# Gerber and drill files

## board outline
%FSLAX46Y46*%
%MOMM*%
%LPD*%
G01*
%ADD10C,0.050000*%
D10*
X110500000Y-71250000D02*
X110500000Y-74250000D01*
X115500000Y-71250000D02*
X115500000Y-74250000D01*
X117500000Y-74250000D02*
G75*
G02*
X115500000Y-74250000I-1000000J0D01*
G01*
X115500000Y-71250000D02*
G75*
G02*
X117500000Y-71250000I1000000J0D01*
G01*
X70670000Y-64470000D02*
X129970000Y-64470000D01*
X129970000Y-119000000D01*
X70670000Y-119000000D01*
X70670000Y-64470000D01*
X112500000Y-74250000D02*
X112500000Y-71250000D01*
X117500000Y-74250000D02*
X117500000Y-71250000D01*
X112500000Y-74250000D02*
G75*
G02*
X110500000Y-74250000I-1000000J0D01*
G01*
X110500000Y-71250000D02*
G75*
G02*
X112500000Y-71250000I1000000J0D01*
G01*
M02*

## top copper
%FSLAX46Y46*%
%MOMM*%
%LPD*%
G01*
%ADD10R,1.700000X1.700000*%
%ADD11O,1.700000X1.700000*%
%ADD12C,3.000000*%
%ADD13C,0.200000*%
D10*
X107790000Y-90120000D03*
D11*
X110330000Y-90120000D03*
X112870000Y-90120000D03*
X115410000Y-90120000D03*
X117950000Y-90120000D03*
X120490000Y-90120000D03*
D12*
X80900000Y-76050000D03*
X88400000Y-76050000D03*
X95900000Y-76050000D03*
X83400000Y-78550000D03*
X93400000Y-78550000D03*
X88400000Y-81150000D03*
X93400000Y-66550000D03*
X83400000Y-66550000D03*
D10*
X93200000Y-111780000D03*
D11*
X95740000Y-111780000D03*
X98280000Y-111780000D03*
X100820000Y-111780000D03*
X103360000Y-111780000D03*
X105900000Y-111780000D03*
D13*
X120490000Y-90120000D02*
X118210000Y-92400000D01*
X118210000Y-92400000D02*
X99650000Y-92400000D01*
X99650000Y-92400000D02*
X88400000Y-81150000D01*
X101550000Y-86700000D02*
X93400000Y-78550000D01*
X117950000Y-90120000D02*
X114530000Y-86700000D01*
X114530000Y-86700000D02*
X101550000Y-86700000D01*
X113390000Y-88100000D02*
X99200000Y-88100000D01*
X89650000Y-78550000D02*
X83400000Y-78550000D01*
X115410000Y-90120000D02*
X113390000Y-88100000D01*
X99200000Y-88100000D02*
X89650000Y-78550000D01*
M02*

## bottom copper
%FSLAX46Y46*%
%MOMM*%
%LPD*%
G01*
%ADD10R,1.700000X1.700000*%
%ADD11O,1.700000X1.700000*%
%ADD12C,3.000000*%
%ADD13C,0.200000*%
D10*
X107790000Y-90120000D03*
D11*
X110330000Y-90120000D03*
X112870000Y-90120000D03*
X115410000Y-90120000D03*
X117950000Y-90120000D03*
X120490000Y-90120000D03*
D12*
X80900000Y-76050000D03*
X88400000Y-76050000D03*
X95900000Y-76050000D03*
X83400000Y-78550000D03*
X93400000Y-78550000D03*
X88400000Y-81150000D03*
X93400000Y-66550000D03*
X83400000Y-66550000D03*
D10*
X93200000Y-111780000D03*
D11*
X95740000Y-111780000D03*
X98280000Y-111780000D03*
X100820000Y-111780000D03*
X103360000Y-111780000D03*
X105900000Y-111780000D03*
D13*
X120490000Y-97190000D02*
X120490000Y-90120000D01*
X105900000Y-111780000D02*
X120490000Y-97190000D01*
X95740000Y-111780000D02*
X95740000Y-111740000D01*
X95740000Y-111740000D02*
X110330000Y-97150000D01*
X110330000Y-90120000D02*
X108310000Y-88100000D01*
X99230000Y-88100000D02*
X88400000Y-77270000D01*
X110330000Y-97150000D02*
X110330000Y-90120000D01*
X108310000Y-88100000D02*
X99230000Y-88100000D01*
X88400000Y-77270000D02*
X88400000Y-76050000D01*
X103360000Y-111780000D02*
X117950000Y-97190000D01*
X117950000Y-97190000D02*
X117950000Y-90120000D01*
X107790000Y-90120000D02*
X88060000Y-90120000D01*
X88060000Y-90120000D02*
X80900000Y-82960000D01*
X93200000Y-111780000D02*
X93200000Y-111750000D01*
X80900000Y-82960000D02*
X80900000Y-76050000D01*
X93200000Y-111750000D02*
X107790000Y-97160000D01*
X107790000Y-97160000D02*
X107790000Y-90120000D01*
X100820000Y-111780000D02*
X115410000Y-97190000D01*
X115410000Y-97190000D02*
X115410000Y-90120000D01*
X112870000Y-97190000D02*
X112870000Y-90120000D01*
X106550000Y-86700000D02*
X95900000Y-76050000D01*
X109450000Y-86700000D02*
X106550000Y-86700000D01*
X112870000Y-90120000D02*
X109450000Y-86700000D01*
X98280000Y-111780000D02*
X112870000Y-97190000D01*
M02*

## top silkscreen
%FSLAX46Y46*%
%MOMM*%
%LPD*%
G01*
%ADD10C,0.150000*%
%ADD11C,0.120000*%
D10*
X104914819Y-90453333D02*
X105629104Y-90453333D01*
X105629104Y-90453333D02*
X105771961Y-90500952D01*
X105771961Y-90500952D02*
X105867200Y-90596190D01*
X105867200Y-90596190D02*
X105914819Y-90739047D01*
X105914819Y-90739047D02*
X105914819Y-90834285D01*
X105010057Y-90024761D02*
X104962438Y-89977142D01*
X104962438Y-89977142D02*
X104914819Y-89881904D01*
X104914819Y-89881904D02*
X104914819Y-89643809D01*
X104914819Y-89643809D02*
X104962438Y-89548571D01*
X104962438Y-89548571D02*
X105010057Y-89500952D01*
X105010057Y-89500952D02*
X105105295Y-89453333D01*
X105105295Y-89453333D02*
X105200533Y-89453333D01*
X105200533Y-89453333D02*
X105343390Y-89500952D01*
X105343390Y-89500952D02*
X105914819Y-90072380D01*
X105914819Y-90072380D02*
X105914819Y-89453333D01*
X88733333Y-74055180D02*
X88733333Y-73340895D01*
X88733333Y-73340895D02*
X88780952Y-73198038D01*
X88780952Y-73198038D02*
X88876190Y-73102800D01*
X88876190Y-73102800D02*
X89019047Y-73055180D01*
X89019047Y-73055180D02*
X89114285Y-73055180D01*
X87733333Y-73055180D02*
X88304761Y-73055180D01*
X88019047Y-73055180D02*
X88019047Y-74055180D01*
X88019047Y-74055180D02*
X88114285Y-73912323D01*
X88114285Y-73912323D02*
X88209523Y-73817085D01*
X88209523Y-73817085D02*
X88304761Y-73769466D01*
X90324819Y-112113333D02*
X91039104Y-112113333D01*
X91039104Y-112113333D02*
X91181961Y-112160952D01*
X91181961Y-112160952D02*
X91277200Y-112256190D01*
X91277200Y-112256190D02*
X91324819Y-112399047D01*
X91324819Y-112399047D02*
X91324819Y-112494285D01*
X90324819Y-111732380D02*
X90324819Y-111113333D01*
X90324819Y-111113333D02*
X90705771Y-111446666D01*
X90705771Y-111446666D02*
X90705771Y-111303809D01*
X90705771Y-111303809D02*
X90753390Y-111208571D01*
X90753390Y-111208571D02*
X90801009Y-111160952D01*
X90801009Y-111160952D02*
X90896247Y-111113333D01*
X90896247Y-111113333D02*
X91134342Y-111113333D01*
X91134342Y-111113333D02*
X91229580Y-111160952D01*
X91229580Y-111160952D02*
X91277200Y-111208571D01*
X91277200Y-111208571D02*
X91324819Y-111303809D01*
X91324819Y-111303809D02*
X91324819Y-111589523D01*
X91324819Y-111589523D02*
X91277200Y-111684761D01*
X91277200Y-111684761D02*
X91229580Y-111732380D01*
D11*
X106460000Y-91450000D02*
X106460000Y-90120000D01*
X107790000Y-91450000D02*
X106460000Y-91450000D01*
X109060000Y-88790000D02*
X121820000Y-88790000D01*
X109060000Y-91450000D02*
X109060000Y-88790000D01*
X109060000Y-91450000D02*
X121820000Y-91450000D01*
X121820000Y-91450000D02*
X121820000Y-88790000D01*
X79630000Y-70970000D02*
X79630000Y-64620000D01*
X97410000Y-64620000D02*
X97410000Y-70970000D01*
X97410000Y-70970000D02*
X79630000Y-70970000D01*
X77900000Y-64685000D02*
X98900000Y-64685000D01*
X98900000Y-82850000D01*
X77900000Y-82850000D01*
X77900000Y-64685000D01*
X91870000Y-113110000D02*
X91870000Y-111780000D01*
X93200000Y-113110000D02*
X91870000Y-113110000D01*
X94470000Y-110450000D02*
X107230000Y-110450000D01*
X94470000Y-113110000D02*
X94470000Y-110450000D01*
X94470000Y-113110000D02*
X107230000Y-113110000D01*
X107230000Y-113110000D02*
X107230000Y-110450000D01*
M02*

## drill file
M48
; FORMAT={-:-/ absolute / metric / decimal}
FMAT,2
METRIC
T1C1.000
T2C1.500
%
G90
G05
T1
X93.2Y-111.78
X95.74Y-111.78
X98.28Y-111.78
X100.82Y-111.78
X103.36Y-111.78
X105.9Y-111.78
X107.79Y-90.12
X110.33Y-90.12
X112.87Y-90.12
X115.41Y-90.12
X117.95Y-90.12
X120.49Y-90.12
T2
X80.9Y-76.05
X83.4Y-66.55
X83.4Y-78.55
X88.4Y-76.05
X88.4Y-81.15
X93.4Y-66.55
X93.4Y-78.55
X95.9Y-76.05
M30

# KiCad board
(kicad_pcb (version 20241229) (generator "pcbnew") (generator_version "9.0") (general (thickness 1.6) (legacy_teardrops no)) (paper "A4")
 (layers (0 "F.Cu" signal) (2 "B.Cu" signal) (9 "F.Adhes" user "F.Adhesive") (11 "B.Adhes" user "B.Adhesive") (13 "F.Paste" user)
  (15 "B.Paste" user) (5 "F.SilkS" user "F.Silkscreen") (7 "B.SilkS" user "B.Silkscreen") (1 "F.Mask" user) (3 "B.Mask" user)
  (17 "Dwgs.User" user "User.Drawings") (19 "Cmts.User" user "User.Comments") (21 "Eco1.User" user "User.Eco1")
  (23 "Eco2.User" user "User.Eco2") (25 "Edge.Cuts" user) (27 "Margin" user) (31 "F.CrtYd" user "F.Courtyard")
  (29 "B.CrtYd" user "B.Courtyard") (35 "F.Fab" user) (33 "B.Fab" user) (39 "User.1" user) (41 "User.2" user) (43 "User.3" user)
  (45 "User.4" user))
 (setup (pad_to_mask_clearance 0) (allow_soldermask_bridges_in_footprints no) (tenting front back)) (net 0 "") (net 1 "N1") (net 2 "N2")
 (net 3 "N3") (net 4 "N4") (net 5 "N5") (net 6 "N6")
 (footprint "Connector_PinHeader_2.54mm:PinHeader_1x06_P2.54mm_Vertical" (layer "F.Cu") (at 107.79 90.12 90)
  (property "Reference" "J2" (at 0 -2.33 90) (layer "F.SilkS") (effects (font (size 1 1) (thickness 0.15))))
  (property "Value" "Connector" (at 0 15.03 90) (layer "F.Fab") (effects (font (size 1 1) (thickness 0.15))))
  (fp_line (start -1.33 -1.33) (end 0 -1.33) (stroke (width 0.12) (type solid)) (layer "F.SilkS"))
  (fp_line (start -1.33 0) (end -1.33 -1.33) (stroke (width 0.12) (type solid)) (layer "F.SilkS"))
  (fp_line (start 1.33 1.27) (end 1.33 14.03) (stroke (width 0.12) (type solid)) (layer "F.SilkS"))
  (fp_line (start -1.33 1.27) (end 1.33 1.27) (stroke (width 0.12) (type solid)) (layer "F.SilkS"))
  (fp_line (start -1.33 1.27) (end -1.33 14.03) (stroke (width 0.12) (type solid)) (layer "F.SilkS"))
  (fp_line (start -1.33 14.03) (end 1.33 14.03) (stroke (width 0.12) (type solid)) (layer "F.SilkS"))
  (pad "1" thru_hole rect (at 0 0 90) (size 1.7 1.7) (drill 1) (layers "*.Cu" "*.Mask") (remove_unused_layers no) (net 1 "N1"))
  (pad "2" thru_hole oval (at 0 2.54 90) (size 1.7 1.7) (drill 1) (layers "*.Cu" "*.Mask") (remove_unused_layers no) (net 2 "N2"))
  (pad "3" thru_hole oval (at 0 5.08 90) (size 1.7 1.7) (drill 1) (layers "*.Cu" "*.Mask") (remove_unused_layers no) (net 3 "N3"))
  (pad "4" thru_hole oval (at 0 7.62 90) (size 1.7 1.7) (drill 1) (layers "*.Cu" "*.Mask") (remove_unused_layers no) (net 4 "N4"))
  (pad "5" thru_hole oval (at 0 10.16 90) (size 1.7 1.7) (drill 1) (layers "*.Cu" "*.Mask") (remove_unused_layers no) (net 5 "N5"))
  (pad "6" thru_hole oval (at 0 12.7 90) (size 1.7 1.7) (drill 1) (layers "*.Cu" "*.Mask") (remove_unused_layers no) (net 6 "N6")))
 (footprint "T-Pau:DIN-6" (layer "F.Cu") (at 80.9 76.05 180)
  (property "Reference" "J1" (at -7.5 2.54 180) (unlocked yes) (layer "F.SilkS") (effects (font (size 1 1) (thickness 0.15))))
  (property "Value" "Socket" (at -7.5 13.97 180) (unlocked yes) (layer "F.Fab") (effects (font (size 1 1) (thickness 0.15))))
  (fp_line (start 1.27 5.08) (end 1.27 11.43) (stroke (width 0.12) (type default)) (layer "F.SilkS"))
  (fp_line (start -16.51 11.43) (end -16.51 5.08) (stroke (width 0.12) (type default)) (layer "F.SilkS"))
  (fp_line (start -16.51 5.08) (end 1.27 5.08) (stroke (width 0.12) (type default)) (layer "F.SilkS"))
  (fp_rect (start -18 -6.8) (end 3 11.365) (stroke (width 0.12) (type default)) (fill no) (layer "F.SilkS"))
  (pad "1" thru_hole circle (at 0 0 180) (size 3 3) (drill 1.5) (layers "*.Cu" "*.Mask") (remove_unused_layers no) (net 1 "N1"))
  (pad "2" thru_hole circle (at -7.5 0 180) (size 3 3) (drill 1.5) (layers "*.Cu" "*.Mask") (remove_unused_layers no) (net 2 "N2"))
  (pad "3" thru_hole circle (at -15 0 180) (size 3 3) (drill 1.5) (layers "*.Cu" "*.Mask") (remove_unused_layers no) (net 3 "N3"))
  (pad "4" thru_hole circle (at -2.5 -2.5 180) (size 3 3) (drill 1.5) (layers "*.Cu" "*.Mask") (remove_unused_layers no) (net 4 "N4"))
  (pad "5" thru_hole circle (at -12.5 -2.5 180) (size 3 3) (drill 1.5) (layers "*.Cu" "*.Mask") (remove_unused_layers no) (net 5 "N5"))
  (pad "6" thru_hole circle (at -7.5 -5.1 180) (size 3 3) (drill 1.5) (layers "*.Cu" "*.Mask") (remove_unused_layers no) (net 6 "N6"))
  (pad "7" thru_hole circle (at -12.5 9.5 180) (size 3 3) (drill 1.5) (layers "*.Cu" "*.Mask") (remove_unused_layers no))
  (pad "7" thru_hole circle (at -2.5 9.5 180) (size 3 3) (drill 1.5) (layers "*.Cu" "*.Mask") (remove_unused_layers no)))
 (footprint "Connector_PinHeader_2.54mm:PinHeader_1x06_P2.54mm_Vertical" (layer "F.Cu") (at 93.2 111.78 90)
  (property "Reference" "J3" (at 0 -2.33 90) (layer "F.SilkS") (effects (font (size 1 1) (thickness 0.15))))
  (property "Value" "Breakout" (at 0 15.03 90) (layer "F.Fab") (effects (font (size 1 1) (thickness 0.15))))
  (fp_line (start -1.33 -1.33) (end 0 -1.33) (stroke (width 0.12) (type solid)) (layer "F.SilkS"))
  (fp_line (start -1.33 0) (end -1.33 -1.33) (stroke (width 0.12) (type solid)) (layer "F.SilkS"))
  (fp_line (start 1.33 1.27) (end 1.33 14.03) (stroke (width 0.12) (type solid)) (layer "F.SilkS"))
  (fp_line (start -1.33 1.27) (end 1.33 1.27) (stroke (width 0.12) (type solid)) (layer "F.SilkS"))
  (fp_line (start -1.33 1.27) (end -1.33 14.03) (stroke (width 0.12) (type solid)) (layer "F.SilkS"))
  (fp_line (start -1.33 14.03) (end 1.33 14.03) (stroke (width 0.12) (type solid)) (layer "F.SilkS"))
  (pad "1" thru_hole rect (at 0 0 90) (size 1.7 1.7) (drill 1) (layers "*.Cu" "*.Mask") (remove_unused_layers no) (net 1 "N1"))
  (pad "2" thru_hole oval (at 0 2.54 90) (size 1.7 1.7) (drill 1) (layers "*.Cu" "*.Mask") (remove_unused_layers no) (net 2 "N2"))
  (pad "3" thru_hole oval (at 0 5.08 90) (size 1.7 1.7) (drill 1) (layers "*.Cu" "*.Mask") (remove_unused_layers no) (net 3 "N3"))
  (pad "4" thru_hole oval (at 0 7.62 90) (size 1.7 1.7) (drill 1) (layers "*.Cu" "*.Mask") (remove_unused_layers no) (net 4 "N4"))
  (pad "5" thru_hole oval (at 0 10.16 90) (size 1.7 1.7) (drill 1) (layers "*.Cu" "*.Mask") (remove_unused_layers no) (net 5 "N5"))
  (pad "6" thru_hole oval (at 0 12.7 90) (size 1.7 1.7) (drill 1) (layers "*.Cu" "*.Mask") (remove_unused_layers no) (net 6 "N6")))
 (gr_line (start 110.5 71.25) (end 110.5 74.25) (stroke (width 0.05) (type default)) (layer "Edge.Cuts"))
 (gr_line (start 115.5 71.25) (end 115.5 74.25) (stroke (width 0.05) (type default)) (layer "Edge.Cuts"))
 (gr_arc (start 117.5 74.25) (mid 116.5 75.25) (end 115.5 74.25) (stroke (width 0.05) (type default)) (layer "Edge.Cuts"))
 (gr_arc (start 115.5 71.25) (mid 116.5 70.25) (end 117.5 71.25) (stroke (width 0.05) (type default)) (layer "Edge.Cuts"))
 (gr_rect (start 70.67 64.47) (end 129.97 119) (stroke (width 0.05) (type default)) (fill no) (layer "Edge.Cuts"))
 (gr_line (start 112.5 74.25) (end 112.5 71.25) (stroke (width 0.05) (type default)) (layer "Edge.Cuts"))
 (gr_line (start 117.5 74.25) (end 117.5 71.25) (stroke (width 0.05) (type default)) (layer "Edge.Cuts"))
 (gr_arc (start 112.5 74.25) (mid 111.5 75.25) (end 110.5 74.25) (stroke (width 0.05) (type default)) (layer "Edge.Cuts"))
 (gr_arc (start 110.5 71.25) (mid 111.5 70.25) (end 112.5 71.25) (stroke (width 0.05) (type default)) (layer "Edge.Cuts"))
 (segment (start 120.49 90.12) (end 118.21 92.4) (width 0.2) (layer "F.Cu") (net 6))
 (segment (start 118.21 92.4) (end 99.65 92.4) (width 0.2) (layer "F.Cu") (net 6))
 (segment (start 99.65 92.4) (end 88.4 81.15) (width 0.2) (layer "F.Cu") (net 6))
 (segment (start 120.49 97.19) (end 120.49 90.12) (width 0.2) (layer "B.Cu") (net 6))
 (segment (start 105.9 111.78) (end 120.49 97.19) (width 0.2) (layer "B.Cu") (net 6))
 (segment (start 95.74 111.78) (end 95.74 111.74) (width 0.2) (layer "B.Cu") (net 2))
 (segment (start 95.74 111.74) (end 110.33 97.15) (width 0.2) (layer "B.Cu") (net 2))
 (segment (start 110.33 90.12) (end 108.31 88.1) (width 0.2) (layer "B.Cu") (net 2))
 (segment (start 99.23 88.1) (end 88.4 77.27) (width 0.2) (layer "B.Cu") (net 2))
 (segment (start 110.33 97.15) (end 110.33 90.12) (width 0.2) (layer "B.Cu") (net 2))
 (segment (start 108.31 88.1) (end 99.23 88.1) (width 0.2) (layer "B.Cu") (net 2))
 (segment (start 88.4 77.27) (end 88.4 76.05) (width 0.2) (layer "B.Cu") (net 2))
 (segment (start 101.55 86.7) (end 93.4 78.55) (width 0.2) (layer "F.Cu") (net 5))
 (segment (start 117.95 90.12) (end 114.53 86.7) (width 0.2) (layer "F.Cu") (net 5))
 (segment (start 114.53 86.7) (end 101.55 86.7) (width 0.2) (layer "F.Cu") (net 5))
 (segment (start 103.36 111.78) (end 117.95 97.19) (width 0.2) (layer "B.Cu") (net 5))
 (segment (start 117.95 97.19) (end 117.95 90.12) (width 0.2) (layer "B.Cu") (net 5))
 (segment (start 107.79 90.12) (end 88.06 90.12) (width 0.2) (layer "B.Cu") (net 1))
 (segment (start 88.06 90.12) (end 80.9 82.96) (width 0.2) (layer "B.Cu") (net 1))
 (segment (start 93.2 111.78) (end 93.2 111.75) (width 0.2) (layer "B.Cu") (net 1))
 (segment (start 80.9 82.96) (end 80.9 76.05) (width 0.2) (layer "B.Cu") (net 1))
 (segment (start 93.2 111.75) (end 107.79 97.16) (width 0.2) (layer "B.Cu") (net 1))
 (segment (start 107.79 97.16) (end 107.79 90.12) (width 0.2) (layer "B.Cu") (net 1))
 (segment (start 113.39 88.1) (end 99.2 88.1) (width 0.2) (layer "F.Cu") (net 4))
 (segment (start 89.65 78.55) (end 83.4 78.55) (width 0.2) (layer "F.Cu") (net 4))
 (segment (start 115.41 90.12) (end 113.39 88.1) (width 0.2) (layer "F.Cu") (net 4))
 (segment (start 99.2 88.1) (end 89.65 78.55) (width 0.2) (layer "F.Cu") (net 4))
 (segment (start 100.82 111.78) (end 115.41 97.19) (width 0.2) (layer "B.Cu") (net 4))
 (segment (start 115.41 97.19) (end 115.41 90.12) (width 0.2) (layer "B.Cu") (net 4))
 (segment (start 112.87 97.19) (end 112.87 90.12) (width 0.2) (layer "B.Cu") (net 3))
 (segment (start 106.55 86.7) (end 95.9 76.05) (width 0.2) (layer "B.Cu") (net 3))
 (segment (start 109.45 86.7) (end 106.55 86.7) (width 0.2) (layer "B.Cu") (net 3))
 (segment (start 112.87 90.12) (end 109.45 86.7) (width 0.2) (layer "B.Cu") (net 3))
 (segment (start 98.28 111.78) (end 112.87 97.19) (width 0.2) (layer "B.Cu") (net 3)))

